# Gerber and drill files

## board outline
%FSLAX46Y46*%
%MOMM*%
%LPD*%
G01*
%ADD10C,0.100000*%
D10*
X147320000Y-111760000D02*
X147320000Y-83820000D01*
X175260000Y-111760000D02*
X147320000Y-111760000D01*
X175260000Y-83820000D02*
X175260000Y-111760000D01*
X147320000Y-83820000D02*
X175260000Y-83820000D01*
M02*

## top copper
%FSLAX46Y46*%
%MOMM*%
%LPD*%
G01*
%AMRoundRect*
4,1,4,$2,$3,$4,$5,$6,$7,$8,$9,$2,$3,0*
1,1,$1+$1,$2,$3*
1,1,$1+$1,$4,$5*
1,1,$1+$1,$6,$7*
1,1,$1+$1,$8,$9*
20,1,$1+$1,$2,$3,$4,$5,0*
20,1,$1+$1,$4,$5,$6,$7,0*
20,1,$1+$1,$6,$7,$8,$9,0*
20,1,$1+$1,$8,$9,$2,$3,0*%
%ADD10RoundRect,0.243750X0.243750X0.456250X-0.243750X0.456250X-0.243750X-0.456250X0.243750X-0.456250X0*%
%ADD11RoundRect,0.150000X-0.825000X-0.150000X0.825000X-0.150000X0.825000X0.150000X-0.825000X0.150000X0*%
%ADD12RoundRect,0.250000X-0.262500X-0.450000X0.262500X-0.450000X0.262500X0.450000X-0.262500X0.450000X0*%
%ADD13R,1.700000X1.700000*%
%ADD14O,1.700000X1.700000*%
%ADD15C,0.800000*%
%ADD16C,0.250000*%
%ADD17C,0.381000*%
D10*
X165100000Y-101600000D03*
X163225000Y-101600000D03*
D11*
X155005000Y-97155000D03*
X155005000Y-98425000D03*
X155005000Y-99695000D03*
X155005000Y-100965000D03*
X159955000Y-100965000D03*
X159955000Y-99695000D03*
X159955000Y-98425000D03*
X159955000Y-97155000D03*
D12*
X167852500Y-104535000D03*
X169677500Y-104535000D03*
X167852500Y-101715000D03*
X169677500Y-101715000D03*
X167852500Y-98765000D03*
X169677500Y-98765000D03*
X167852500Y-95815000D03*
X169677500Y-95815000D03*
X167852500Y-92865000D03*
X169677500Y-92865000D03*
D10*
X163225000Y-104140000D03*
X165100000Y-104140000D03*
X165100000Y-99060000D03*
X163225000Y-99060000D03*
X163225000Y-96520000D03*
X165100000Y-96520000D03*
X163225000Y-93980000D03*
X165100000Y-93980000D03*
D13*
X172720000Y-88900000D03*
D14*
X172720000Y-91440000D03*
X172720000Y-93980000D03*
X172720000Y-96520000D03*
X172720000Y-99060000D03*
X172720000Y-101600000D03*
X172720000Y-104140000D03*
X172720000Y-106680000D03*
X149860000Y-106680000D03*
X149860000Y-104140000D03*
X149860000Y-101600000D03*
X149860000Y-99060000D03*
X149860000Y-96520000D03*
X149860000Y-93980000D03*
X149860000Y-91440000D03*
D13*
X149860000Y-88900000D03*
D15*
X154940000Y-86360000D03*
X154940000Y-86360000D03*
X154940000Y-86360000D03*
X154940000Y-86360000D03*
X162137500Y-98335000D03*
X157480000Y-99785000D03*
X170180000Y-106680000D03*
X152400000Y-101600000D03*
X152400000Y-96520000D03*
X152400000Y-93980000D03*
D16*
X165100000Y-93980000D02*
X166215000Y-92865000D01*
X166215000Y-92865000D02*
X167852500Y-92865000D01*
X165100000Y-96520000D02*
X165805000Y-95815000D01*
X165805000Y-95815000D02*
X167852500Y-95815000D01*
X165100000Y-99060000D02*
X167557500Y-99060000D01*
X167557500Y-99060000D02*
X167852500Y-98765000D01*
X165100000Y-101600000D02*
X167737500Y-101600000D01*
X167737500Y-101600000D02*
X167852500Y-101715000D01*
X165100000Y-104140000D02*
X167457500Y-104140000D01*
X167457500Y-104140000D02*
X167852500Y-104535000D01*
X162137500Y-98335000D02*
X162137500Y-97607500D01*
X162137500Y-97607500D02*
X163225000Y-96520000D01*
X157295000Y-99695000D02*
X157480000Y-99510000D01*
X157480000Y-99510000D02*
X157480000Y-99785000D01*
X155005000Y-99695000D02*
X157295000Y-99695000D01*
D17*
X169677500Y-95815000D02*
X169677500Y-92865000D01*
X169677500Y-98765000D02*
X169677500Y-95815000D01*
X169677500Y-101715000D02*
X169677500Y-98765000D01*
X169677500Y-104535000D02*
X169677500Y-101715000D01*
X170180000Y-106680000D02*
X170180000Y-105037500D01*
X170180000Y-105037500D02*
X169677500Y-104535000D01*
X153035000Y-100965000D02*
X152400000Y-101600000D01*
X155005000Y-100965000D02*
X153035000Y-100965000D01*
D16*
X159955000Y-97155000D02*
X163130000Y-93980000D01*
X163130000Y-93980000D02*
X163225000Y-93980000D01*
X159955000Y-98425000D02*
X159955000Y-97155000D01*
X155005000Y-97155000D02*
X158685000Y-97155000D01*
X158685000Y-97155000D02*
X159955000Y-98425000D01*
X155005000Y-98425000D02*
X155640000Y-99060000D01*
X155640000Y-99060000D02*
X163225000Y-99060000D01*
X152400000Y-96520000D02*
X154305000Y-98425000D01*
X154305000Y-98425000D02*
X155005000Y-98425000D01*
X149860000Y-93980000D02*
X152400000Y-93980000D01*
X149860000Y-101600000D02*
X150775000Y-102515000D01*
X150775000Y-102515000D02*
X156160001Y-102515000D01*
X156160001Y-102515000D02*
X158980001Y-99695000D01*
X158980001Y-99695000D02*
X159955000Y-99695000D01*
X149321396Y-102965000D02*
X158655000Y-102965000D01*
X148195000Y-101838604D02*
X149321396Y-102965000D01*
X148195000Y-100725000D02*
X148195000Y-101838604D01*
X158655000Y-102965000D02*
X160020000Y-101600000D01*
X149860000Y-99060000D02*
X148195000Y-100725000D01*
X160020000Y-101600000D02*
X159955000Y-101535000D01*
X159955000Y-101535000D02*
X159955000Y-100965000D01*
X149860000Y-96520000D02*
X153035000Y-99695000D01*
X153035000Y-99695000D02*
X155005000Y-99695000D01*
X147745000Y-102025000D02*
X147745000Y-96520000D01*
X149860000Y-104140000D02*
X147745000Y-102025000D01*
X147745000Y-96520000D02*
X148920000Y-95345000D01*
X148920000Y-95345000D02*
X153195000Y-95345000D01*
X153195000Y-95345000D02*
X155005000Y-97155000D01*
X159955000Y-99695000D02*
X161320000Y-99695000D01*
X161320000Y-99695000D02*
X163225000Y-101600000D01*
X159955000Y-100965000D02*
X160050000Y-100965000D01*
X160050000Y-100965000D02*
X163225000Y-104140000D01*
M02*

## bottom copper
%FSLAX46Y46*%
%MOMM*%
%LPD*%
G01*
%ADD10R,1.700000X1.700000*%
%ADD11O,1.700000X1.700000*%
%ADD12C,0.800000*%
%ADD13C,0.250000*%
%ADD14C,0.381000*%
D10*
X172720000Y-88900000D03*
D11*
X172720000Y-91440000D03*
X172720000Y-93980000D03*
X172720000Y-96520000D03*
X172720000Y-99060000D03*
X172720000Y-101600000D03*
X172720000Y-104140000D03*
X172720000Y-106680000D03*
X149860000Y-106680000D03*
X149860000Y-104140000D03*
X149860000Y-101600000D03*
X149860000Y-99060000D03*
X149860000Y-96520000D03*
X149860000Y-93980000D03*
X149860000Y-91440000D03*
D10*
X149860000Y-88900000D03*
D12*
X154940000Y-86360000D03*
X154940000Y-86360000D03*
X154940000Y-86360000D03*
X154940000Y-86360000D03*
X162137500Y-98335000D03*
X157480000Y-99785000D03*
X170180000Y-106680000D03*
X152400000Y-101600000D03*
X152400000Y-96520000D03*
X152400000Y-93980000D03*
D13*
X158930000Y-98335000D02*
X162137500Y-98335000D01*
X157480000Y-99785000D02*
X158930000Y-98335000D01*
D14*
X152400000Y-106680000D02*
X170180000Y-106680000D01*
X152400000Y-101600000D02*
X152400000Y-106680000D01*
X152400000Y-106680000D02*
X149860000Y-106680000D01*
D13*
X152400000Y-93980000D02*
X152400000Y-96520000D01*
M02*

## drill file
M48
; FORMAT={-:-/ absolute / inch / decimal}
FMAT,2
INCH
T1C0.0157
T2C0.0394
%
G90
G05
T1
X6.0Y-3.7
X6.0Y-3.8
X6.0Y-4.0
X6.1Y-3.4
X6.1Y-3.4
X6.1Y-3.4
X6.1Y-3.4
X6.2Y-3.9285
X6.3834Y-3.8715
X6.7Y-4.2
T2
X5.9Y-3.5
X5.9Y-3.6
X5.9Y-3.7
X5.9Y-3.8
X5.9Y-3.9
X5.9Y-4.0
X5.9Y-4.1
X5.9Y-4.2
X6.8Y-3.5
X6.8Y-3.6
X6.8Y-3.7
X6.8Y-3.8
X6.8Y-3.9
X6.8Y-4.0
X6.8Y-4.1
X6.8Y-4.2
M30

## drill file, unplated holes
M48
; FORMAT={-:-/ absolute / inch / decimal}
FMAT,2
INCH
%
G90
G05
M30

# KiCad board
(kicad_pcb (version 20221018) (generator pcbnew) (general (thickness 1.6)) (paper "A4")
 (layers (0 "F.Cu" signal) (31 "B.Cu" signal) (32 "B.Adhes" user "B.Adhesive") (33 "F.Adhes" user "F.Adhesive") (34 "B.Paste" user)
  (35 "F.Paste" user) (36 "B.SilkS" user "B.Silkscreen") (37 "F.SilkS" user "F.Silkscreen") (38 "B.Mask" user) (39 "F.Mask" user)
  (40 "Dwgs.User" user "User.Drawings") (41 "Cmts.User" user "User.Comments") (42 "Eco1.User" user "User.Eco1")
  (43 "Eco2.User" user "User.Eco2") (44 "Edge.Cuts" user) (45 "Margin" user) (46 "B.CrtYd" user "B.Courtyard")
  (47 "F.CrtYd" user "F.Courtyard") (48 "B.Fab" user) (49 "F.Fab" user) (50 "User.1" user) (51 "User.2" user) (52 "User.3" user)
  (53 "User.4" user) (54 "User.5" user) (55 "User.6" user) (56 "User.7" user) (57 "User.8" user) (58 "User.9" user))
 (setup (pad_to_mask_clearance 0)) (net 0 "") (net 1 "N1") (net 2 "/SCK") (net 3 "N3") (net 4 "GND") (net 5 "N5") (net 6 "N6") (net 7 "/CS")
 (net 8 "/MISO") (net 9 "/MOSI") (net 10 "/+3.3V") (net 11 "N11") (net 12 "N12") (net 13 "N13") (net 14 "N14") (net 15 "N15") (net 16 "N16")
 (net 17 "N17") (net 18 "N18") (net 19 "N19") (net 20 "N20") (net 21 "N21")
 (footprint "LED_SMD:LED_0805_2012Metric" (layer "F.Cu") (at 164.1625 96.52 180)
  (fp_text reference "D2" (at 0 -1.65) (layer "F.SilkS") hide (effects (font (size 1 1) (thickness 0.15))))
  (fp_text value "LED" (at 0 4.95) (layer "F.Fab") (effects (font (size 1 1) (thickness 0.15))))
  (pad "1" smd roundrect (at -0.9375 0 180) (size 0.975 1.4) (layers "F.Cu" "F.Paste" "F.Mask") (roundrect_rratio 0.25) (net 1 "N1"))
  (pad "2" smd roundrect (at 0.9375 0 180) (size 0.975 1.4) (layers "F.Cu" "F.Paste" "F.Mask") (roundrect_rratio 0.25) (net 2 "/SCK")))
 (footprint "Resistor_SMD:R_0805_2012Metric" (layer "F.Cu") (at 168.765 104.535)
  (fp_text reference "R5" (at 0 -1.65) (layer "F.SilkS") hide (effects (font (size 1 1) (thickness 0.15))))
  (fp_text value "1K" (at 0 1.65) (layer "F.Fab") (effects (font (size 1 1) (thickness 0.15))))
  (pad "1" smd roundrect (at -0.9125 0) (size 1.025 1.4) (layers "F.Cu" "F.Paste" "F.Mask") (roundrect_rratio 0.243902439) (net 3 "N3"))
  (pad "2" smd roundrect (at 0.9125 0) (size 1.025 1.4) (layers "F.Cu" "F.Paste" "F.Mask") (roundrect_rratio 0.243902439) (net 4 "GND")))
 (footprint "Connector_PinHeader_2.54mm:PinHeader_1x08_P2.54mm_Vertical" (layer "F.Cu") (at 149.86 88.9)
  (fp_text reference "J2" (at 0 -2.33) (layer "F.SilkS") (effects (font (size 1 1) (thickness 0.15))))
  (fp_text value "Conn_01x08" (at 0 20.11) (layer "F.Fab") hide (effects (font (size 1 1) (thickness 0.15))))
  (pad "1" thru_hole rect (at 0 0) (size 1.7 1.7) (drill 1) (layers "*.Cu" "*.Mask") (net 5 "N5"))
  (pad "2" thru_hole oval (at 0 2.54) (size 1.7 1.7) (drill 1) (layers "*.Cu" "*.Mask") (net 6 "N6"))
  (pad "3" thru_hole oval (at 0 5.08) (size 1.7 1.7) (drill 1) (layers "*.Cu" "*.Mask") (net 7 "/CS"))
  (pad "4" thru_hole oval (at 0 7.62) (size 1.7 1.7) (drill 1) (layers "*.Cu" "*.Mask") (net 2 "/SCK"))
  (pad "5" thru_hole oval (at 0 10.16) (size 1.7 1.7) (drill 1) (layers "*.Cu" "*.Mask") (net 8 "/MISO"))
  (pad "6" thru_hole oval (at 0 12.7) (size 1.7 1.7) (drill 1) (layers "*.Cu" "*.Mask") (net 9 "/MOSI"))
  (pad "7" thru_hole oval (at 0 15.24) (size 1.7 1.7) (drill 1) (layers "*.Cu" "*.Mask") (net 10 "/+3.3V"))
  (pad "8" thru_hole oval (at 0 17.78) (size 1.7 1.7) (drill 1) (layers "*.Cu" "*.Mask") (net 4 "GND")))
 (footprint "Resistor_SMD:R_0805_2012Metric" (layer "F.Cu") (at 168.765 95.815)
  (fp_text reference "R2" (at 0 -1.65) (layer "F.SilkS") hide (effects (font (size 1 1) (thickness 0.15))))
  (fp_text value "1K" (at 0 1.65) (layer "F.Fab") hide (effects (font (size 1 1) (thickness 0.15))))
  (pad "1" smd roundrect (at -0.9125 0) (size 1.025 1.4) (layers "F.Cu" "F.Paste" "F.Mask") (roundrect_rratio 0.243902439) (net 1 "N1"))
  (pad "2" smd roundrect (at 0.9125 0) (size 1.025 1.4) (layers "F.Cu" "F.Paste" "F.Mask") (roundrect_rratio 0.243902439) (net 4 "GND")))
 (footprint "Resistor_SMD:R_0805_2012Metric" (layer "F.Cu") (at 168.765 101.715)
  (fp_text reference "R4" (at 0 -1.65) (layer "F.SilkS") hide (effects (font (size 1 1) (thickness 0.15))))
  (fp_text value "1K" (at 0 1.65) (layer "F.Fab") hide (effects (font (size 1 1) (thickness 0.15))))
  (pad "1" smd roundrect (at -0.9125 0) (size 1.025 1.4) (layers "F.Cu" "F.Paste" "F.Mask") (roundrect_rratio 0.243902439) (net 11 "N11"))
  (pad "2" smd roundrect (at 0.9125 0) (size 1.025 1.4) (layers "F.Cu" "F.Paste" "F.Mask") (roundrect_rratio 0.243902439) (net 4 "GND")))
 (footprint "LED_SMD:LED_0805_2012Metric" (layer "F.Cu") (at 164.1625 99.06 180)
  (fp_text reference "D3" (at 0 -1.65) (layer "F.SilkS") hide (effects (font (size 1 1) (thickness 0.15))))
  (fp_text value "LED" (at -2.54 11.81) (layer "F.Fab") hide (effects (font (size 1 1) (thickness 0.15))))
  (pad "1" smd roundrect (at -0.9375 0 180) (size 0.975 1.4) (layers "F.Cu" "F.Paste" "F.Mask") (roundrect_rratio 0.25) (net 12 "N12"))
  (pad "2" smd roundrect (at 0.9375 0 180) (size 0.975 1.4) (layers "F.Cu" "F.Paste" "F.Mask") (roundrect_rratio 0.25) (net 7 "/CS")))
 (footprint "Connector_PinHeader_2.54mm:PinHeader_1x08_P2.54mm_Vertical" (layer "F.Cu") (at 172.72 88.9)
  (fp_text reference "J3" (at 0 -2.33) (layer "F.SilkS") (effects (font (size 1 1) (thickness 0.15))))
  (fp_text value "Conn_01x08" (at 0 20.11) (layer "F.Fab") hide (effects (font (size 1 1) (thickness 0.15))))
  (pad "1" thru_hole rect (at 0 0) (size 1.7 1.7) (drill 1) (layers "*.Cu" "*.Mask") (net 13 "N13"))
  (pad "2" thru_hole oval (at 0 2.54) (size 1.7 1.7) (drill 1) (layers "*.Cu" "*.Mask") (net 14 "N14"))
  (pad "3" thru_hole oval (at 0 5.08) (size 1.7 1.7) (drill 1) (layers "*.Cu" "*.Mask") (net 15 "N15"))
  (pad "4" thru_hole oval (at 0 7.62) (size 1.7 1.7) (drill 1) (layers "*.Cu" "*.Mask") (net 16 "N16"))
  (pad "5" thru_hole oval (at 0 10.16) (size 1.7 1.7) (drill 1) (layers "*.Cu" "*.Mask") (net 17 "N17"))
  (pad "6" thru_hole oval (at 0 12.7) (size 1.7 1.7) (drill 1) (layers "*.Cu" "*.Mask") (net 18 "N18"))
  (pad "7" thru_hole oval (at 0 15.24) (size 1.7 1.7) (drill 1) (layers "*.Cu" "*.Mask") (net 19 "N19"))
  (pad "8" thru_hole oval (at 0 17.78) (size 1.7 1.7) (drill 1) (layers "*.Cu" "*.Mask") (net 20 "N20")))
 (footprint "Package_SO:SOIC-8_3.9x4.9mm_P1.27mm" (layer "F.Cu") (at 157.48 99.06)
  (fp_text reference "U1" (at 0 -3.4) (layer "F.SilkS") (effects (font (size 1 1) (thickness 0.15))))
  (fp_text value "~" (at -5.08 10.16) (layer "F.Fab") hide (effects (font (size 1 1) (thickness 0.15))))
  (pad "1" smd roundrect (at -2.475 -1.905) (size 1.95 0.6) (layers "F.Cu" "F.Paste" "F.Mask") (roundrect_rratio 0.25) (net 10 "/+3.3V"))
  (pad "2" smd roundrect (at -2.475 -0.635) (size 1.95 0.6) (layers "F.Cu" "F.Paste" "F.Mask") (roundrect_rratio 0.25) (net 7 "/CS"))
  (pad "3" smd roundrect (at -2.475 0.635) (size 1.95 0.6) (layers "F.Cu" "F.Paste" "F.Mask") (roundrect_rratio 0.25) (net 2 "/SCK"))
  (pad "4" smd roundrect (at -2.475 1.905) (size 1.95 0.6) (layers "F.Cu" "F.Paste" "F.Mask") (roundrect_rratio 0.25) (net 4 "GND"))
  (pad "5" smd roundrect (at 2.475 1.905) (size 1.95 0.6) (layers "F.Cu" "F.Paste" "F.Mask") (roundrect_rratio 0.25) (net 8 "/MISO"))
  (pad "6" smd roundrect (at 2.475 0.635) (size 1.95 0.6) (layers "F.Cu" "F.Paste" "F.Mask") (roundrect_rratio 0.25) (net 9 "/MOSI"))
  (pad "7" smd roundrect (at 2.475 -0.635) (size 1.95 0.6) (layers "F.Cu" "F.Paste" "F.Mask") (roundrect_rratio 0.25) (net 10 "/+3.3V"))
  (pad "8" smd roundrect (at 2.475 -1.905) (size 1.95 0.6) (layers "F.Cu" "F.Paste" "F.Mask") (roundrect_rratio 0.25) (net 10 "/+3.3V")))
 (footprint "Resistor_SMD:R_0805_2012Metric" (layer "F.Cu") (at 168.765 92.865)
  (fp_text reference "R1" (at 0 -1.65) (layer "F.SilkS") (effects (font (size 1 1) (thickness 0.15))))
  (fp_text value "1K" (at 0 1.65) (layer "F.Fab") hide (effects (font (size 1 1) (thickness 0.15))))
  (pad "1" smd roundrect (at -0.9125 0) (size 1.025 1.4) (layers "F.Cu" "F.Paste" "F.Mask") (roundrect_rratio 0.243902439) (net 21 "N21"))
  (pad "2" smd roundrect (at 0.9125 0) (size 1.025 1.4) (layers "F.Cu" "F.Paste" "F.Mask") (roundrect_rratio 0.243902439) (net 4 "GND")))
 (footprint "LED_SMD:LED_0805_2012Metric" (layer "F.Cu") (at 164.1625 93.98 180)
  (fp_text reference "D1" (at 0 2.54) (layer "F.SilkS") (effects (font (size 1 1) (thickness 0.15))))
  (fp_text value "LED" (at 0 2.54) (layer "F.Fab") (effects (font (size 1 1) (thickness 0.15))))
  (pad "1" smd roundrect (at -0.9375 0 180) (size 0.975 1.4) (layers "F.Cu" "F.Paste" "F.Mask") (roundrect_rratio 0.25) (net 21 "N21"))
  (pad "2" smd roundrect (at 0.9375 0 180) (size 0.975 1.4) (layers "F.Cu" "F.Paste" "F.Mask") (roundrect_rratio 0.25) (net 10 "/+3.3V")))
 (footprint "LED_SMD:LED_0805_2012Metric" (layer "F.Cu") (at 164.1625 104.14 180)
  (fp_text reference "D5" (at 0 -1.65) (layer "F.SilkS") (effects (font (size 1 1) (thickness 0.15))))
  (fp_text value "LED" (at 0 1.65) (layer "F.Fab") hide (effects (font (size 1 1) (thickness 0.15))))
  (pad "1" smd roundrect (at -0.9375 0 180) (size 0.975 1.4) (layers "F.Cu" "F.Paste" "F.Mask") (roundrect_rratio 0.25) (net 3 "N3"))
  (pad "2" smd roundrect (at 0.9375 0 180) (size 0.975 1.4) (layers "F.Cu" "F.Paste" "F.Mask") (roundrect_rratio 0.25) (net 8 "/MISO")))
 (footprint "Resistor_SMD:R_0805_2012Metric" (layer "F.Cu") (at 168.765 98.765)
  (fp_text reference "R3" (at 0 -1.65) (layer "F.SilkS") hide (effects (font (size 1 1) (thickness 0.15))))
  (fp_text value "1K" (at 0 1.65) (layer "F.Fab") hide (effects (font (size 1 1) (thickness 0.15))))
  (pad "1" smd roundrect (at -0.9125 0) (size 1.025 1.4) (layers "F.Cu" "F.Paste" "F.Mask") (roundrect_rratio 0.243902439) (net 12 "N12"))
  (pad "2" smd roundrect (at 0.9125 0) (size 1.025 1.4) (layers "F.Cu" "F.Paste" "F.Mask") (roundrect_rratio 0.243902439) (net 4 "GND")))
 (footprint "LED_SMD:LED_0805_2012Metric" (layer "F.Cu") (at 164.1625 101.6 180)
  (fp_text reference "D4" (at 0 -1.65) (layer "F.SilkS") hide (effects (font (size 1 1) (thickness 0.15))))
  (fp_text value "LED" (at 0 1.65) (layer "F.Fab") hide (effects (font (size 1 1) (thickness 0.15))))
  (pad "1" smd roundrect (at -0.9375 0 180) (size 0.975 1.4) (layers "F.Cu" "F.Paste" "F.Mask") (roundrect_rratio 0.25) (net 11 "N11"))
  (pad "2" smd roundrect (at 0.9375 0 180) (size 0.975 1.4) (layers "F.Cu" "F.Paste" "F.Mask") (roundrect_rratio 0.25) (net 9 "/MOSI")))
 (gr_line (start 175.26 83.82) (end 175.26 111.76) (stroke (width 0.1) (type default)) (layer "Edge.Cuts"))
 (gr_line (start 147.32 83.82) (end 175.26 83.82) (stroke (width 0.1) (type default)) (layer "Edge.Cuts"))
 (gr_line (start 147.32 111.76) (end 147.32 83.82) (stroke (width 0.1) (type default)) (layer "Edge.Cuts"))
 (gr_line (start 175.26 111.76) (end 147.32 111.76) (stroke (width 0.1) (type default)) (layer "Edge.Cuts"))
 (via (at 154.94 86.36) (size 0.8) (drill 0.4) (layers "F.Cu" "B.Cu") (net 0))
 (via (at 154.94 86.36) (size 0.8) (drill 0.4) (layers "F.Cu" "B.Cu") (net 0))
 (via (at 154.94 86.36) (size 0.8) (drill 0.4) (layers "F.Cu" "B.Cu") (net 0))
 (via (at 154.94 86.36) (size 0.8) (drill 0.4) (layers "F.Cu" "B.Cu") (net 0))
 (segment (start 166.215 92.865) (end 167.8525 92.865) (width 0.25) (layer "F.Cu") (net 21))
 (segment (start 165.1 93.98) (end 166.215 92.865) (width 0.25) (layer "F.Cu") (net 21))
 (segment (start 165.805 95.815) (end 167.8525 95.815) (width 0.25) (layer "F.Cu") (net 1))
 (segment (start 165.1 96.52) (end 165.805 95.815) (width 0.25) (layer "F.Cu") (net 1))
 (segment (start 165.1 99.06) (end 167.5575 99.06) (width 0.25) (layer "F.Cu") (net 12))
 (segment (start 167.5575 99.06) (end 167.8525 98.765) (width 0.25) (layer "F.Cu") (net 12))
 (segment (start 167.7375 101.6) (end 167.8525 101.715) (width 0.25) (layer "F.Cu") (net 11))
 (segment (start 165.1 101.6) (end 167.7375 101.6) (width 0.25) (layer "F.Cu") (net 11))
 (segment (start 165.1 104.14) (end 167.4575 104.14) (width 0.25) (layer "F.Cu") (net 3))
 (segment (start 167.4575 104.14) (end 167.8525 104.535) (width 0.25) (layer "F.Cu") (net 3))
 (segment (start 169.6775 98.765) (end 169.6775 95.815) (width 0.381) (layer "F.Cu") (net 4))
 (segment (start 169.6775 95.815) (end 169.6775 92.865) (width 0.381) (layer "F.Cu") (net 4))
 (segment (start 169.6775 101.715) (end 169.6775 98.765) (width 0.381) (layer "F.Cu") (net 4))
 (segment (start 169.6775 104.535) (end 169.6775 101.715) (width 0.381) (layer "F.Cu") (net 4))
 (segment (start 155.005 100.965) (end 153.035 100.965) (width 0.381) (layer "F.Cu") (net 4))
 (segment (start 170.18 105.0375) (end 169.6775 104.535) (width 0.381) (layer "F.Cu") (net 4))
 (segment (start 153.035 100.965) (end 152.4 101.6) (width 0.381) (layer "F.Cu") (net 4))
 (segment (start 170.18 106.68) (end 170.18 105.0375) (width 0.381) (layer "F.Cu") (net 4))
 (via (at 170.18 106.68) (size 0.8) (drill 0.4) (layers "F.Cu" "B.Cu") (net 4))
 (via (at 152.4 101.6) (size 0.8) (drill 0.4) (layers "F.Cu" "B.Cu") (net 4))
 (segment (start 152.4 101.6) (end 152.4 106.68) (width 0.381) (layer "B.Cu") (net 4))
 (segment (start 152.4 106.68) (end 170.18 106.68) (width 0.381) (layer "B.Cu") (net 4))
 (segment (start 152.4 106.68) (end 149.86 106.68) (width 0.381) (layer "B.Cu") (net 4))
 (segment (start 152.4 96.52) (end 154.305 98.425) (width 0.25) (layer "F.Cu") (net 7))
 (segment (start 149.86 93.98) (end 152.4 93.98) (width 0.25) (layer "F.Cu") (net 7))
 (segment (start 154.305 98.425) (end 155.005 98.425) (width 0.25) (layer "F.Cu") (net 7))
 (segment (start 155.64 99.06) (end 163.225 99.06) (width 0.25) (layer "F.Cu") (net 7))
 (segment (start 155.005 98.425) (end 155.64 99.06) (width 0.25) (layer "F.Cu") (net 7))
 (via (at 152.4 96.52) (size 0.8) (drill 0.4) (layers "F.Cu" "B.Cu") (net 7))
 (via (at 152.4 93.98) (size 0.8) (drill 0.4) (layers "F.Cu" "B.Cu") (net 7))
 (segment (start 152.4 93.98) (end 152.4 96.52) (width 0.25) (layer "B.Cu") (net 7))
 (segment (start 162.1375 98.335) (end 162.1375 97.6075) (width 0.25) (layer "F.Cu") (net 2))
 (segment (start 162.1375 97.6075) (end 163.225 96.52) (width 0.25) (layer "F.Cu") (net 2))
 (segment (start 157.295 99.695) (end 157.48 99.51) (width 0.25) (layer "F.Cu") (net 2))
 (segment (start 155.005 99.695) (end 157.295 99.695) (width 0.25) (layer "F.Cu") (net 2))
 (segment (start 157.48 99.51) (end 157.48 99.785) (width 0.25) (layer "F.Cu") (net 2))
 (segment (start 153.035 99.695) (end 155.005 99.695) (width 0.25) (layer "F.Cu") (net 2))
 (segment (start 149.86 96.52) (end 153.035 99.695) (width 0.25) (layer "F.Cu") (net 2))
 (via (at 157.48 99.785) (size 0.8) (drill 0.4) (layers "F.Cu" "B.Cu") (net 2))
 (via (at 162.1375 98.335) (size 0.8) (drill 0.4) (layers "F.Cu" "B.Cu") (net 2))
 (segment (start 158.93 98.335) (end 162.1375 98.335) (width 0.25) (layer "B.Cu") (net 2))
 (segment (start 157.48 99.785) (end 158.93 98.335) (width 0.25) (layer "B.Cu") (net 2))
 (segment (start 158.655 102.965) (end 160.02 101.6) (width 0.25) (layer "F.Cu") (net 8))
 (segment (start 148.195 101.838604) (end 149.321396 102.965) (width 0.25) (layer "F.Cu") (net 8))
 (segment (start 149.86 99.06) (end 148.195 100.725) (width 0.25) (layer "F.Cu") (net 8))
 (segment (start 148.195 100.725) (end 148.195 101.838604) (width 0.25) (layer "F.Cu") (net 8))
 (segment (start 159.955 100.965) (end 160.05 100.965) (width 0.25) (layer "F.Cu") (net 8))
 (segment (start 159.955 101.535) (end 159.955 100.965) (width 0.25) (layer "F.Cu") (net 8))
 (segment (start 160.05 100.965) (end 163.225 104.14) (width 0.25) (layer "F.Cu") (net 8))
 (segment (start 160.02 101.6) (end 159.955 101.535) (width 0.25) (layer "F.Cu") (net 8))
 (segment (start 149.321396 102.965) (end 158.655 102.965) (width 0.25) (layer "F.Cu") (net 8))
 (segment (start 156.160001 102.515) (end 158.980001 99.695) (width 0.25) (layer "F.Cu") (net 9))
 (segment (start 158.980001 99.695) (end 159.955 99.695) (width 0.25) (layer "F.Cu") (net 9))
 (segment (start 150.775 102.515) (end 156.160001 102.515) (width 0.25) (layer "F.Cu") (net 9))
 (segment (start 161.32 99.695) (end 163.225 101.6) (width 0.25) (layer "F.Cu") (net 9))
 (segment (start 159.955 99.695) (end 161.32 99.695) (width 0.25) (layer "F.Cu") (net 9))
 (segment (start 149.86 101.6) (end 150.775 102.515) (width 0.25) (layer "F.Cu") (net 9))
 (segment (start 159.955 98.425) (end 159.955 97.155) (width 0.25) (layer "F.Cu") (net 10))
 (segment (start 147.745 102.025) (end 147.745 96.52) (width 0.25) (layer "F.Cu") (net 10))
 (segment (start 159.955 97.155) (end 163.13 93.98) (width 0.25) (layer "F.Cu") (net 10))
 (segment (start 147.745 96.52) (end 148.92 95.345) (width 0.25) (layer "F.Cu") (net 10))
 (segment (start 155.005 97.155) (end 158.685 97.155) (width 0.25) (layer "F.Cu") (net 10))
 (segment (start 149.86 104.14) (end 147.745 102.025) (width 0.25) (layer "F.Cu") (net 10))
 (segment (start 148.92 95.345) (end 153.195 95.345) (width 0.25) (layer "F.Cu") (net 10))
 (segment (start 163.13 93.98) (end 163.225 93.98) (width 0.25) (layer "F.Cu") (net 10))
 (segment (start 153.195 95.345) (end 155.005 97.155) (width 0.25) (layer "F.Cu") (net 10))
 (segment (start 158.685 97.155) (end 159.955 98.425) (width 0.25) (layer "F.Cu") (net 10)))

